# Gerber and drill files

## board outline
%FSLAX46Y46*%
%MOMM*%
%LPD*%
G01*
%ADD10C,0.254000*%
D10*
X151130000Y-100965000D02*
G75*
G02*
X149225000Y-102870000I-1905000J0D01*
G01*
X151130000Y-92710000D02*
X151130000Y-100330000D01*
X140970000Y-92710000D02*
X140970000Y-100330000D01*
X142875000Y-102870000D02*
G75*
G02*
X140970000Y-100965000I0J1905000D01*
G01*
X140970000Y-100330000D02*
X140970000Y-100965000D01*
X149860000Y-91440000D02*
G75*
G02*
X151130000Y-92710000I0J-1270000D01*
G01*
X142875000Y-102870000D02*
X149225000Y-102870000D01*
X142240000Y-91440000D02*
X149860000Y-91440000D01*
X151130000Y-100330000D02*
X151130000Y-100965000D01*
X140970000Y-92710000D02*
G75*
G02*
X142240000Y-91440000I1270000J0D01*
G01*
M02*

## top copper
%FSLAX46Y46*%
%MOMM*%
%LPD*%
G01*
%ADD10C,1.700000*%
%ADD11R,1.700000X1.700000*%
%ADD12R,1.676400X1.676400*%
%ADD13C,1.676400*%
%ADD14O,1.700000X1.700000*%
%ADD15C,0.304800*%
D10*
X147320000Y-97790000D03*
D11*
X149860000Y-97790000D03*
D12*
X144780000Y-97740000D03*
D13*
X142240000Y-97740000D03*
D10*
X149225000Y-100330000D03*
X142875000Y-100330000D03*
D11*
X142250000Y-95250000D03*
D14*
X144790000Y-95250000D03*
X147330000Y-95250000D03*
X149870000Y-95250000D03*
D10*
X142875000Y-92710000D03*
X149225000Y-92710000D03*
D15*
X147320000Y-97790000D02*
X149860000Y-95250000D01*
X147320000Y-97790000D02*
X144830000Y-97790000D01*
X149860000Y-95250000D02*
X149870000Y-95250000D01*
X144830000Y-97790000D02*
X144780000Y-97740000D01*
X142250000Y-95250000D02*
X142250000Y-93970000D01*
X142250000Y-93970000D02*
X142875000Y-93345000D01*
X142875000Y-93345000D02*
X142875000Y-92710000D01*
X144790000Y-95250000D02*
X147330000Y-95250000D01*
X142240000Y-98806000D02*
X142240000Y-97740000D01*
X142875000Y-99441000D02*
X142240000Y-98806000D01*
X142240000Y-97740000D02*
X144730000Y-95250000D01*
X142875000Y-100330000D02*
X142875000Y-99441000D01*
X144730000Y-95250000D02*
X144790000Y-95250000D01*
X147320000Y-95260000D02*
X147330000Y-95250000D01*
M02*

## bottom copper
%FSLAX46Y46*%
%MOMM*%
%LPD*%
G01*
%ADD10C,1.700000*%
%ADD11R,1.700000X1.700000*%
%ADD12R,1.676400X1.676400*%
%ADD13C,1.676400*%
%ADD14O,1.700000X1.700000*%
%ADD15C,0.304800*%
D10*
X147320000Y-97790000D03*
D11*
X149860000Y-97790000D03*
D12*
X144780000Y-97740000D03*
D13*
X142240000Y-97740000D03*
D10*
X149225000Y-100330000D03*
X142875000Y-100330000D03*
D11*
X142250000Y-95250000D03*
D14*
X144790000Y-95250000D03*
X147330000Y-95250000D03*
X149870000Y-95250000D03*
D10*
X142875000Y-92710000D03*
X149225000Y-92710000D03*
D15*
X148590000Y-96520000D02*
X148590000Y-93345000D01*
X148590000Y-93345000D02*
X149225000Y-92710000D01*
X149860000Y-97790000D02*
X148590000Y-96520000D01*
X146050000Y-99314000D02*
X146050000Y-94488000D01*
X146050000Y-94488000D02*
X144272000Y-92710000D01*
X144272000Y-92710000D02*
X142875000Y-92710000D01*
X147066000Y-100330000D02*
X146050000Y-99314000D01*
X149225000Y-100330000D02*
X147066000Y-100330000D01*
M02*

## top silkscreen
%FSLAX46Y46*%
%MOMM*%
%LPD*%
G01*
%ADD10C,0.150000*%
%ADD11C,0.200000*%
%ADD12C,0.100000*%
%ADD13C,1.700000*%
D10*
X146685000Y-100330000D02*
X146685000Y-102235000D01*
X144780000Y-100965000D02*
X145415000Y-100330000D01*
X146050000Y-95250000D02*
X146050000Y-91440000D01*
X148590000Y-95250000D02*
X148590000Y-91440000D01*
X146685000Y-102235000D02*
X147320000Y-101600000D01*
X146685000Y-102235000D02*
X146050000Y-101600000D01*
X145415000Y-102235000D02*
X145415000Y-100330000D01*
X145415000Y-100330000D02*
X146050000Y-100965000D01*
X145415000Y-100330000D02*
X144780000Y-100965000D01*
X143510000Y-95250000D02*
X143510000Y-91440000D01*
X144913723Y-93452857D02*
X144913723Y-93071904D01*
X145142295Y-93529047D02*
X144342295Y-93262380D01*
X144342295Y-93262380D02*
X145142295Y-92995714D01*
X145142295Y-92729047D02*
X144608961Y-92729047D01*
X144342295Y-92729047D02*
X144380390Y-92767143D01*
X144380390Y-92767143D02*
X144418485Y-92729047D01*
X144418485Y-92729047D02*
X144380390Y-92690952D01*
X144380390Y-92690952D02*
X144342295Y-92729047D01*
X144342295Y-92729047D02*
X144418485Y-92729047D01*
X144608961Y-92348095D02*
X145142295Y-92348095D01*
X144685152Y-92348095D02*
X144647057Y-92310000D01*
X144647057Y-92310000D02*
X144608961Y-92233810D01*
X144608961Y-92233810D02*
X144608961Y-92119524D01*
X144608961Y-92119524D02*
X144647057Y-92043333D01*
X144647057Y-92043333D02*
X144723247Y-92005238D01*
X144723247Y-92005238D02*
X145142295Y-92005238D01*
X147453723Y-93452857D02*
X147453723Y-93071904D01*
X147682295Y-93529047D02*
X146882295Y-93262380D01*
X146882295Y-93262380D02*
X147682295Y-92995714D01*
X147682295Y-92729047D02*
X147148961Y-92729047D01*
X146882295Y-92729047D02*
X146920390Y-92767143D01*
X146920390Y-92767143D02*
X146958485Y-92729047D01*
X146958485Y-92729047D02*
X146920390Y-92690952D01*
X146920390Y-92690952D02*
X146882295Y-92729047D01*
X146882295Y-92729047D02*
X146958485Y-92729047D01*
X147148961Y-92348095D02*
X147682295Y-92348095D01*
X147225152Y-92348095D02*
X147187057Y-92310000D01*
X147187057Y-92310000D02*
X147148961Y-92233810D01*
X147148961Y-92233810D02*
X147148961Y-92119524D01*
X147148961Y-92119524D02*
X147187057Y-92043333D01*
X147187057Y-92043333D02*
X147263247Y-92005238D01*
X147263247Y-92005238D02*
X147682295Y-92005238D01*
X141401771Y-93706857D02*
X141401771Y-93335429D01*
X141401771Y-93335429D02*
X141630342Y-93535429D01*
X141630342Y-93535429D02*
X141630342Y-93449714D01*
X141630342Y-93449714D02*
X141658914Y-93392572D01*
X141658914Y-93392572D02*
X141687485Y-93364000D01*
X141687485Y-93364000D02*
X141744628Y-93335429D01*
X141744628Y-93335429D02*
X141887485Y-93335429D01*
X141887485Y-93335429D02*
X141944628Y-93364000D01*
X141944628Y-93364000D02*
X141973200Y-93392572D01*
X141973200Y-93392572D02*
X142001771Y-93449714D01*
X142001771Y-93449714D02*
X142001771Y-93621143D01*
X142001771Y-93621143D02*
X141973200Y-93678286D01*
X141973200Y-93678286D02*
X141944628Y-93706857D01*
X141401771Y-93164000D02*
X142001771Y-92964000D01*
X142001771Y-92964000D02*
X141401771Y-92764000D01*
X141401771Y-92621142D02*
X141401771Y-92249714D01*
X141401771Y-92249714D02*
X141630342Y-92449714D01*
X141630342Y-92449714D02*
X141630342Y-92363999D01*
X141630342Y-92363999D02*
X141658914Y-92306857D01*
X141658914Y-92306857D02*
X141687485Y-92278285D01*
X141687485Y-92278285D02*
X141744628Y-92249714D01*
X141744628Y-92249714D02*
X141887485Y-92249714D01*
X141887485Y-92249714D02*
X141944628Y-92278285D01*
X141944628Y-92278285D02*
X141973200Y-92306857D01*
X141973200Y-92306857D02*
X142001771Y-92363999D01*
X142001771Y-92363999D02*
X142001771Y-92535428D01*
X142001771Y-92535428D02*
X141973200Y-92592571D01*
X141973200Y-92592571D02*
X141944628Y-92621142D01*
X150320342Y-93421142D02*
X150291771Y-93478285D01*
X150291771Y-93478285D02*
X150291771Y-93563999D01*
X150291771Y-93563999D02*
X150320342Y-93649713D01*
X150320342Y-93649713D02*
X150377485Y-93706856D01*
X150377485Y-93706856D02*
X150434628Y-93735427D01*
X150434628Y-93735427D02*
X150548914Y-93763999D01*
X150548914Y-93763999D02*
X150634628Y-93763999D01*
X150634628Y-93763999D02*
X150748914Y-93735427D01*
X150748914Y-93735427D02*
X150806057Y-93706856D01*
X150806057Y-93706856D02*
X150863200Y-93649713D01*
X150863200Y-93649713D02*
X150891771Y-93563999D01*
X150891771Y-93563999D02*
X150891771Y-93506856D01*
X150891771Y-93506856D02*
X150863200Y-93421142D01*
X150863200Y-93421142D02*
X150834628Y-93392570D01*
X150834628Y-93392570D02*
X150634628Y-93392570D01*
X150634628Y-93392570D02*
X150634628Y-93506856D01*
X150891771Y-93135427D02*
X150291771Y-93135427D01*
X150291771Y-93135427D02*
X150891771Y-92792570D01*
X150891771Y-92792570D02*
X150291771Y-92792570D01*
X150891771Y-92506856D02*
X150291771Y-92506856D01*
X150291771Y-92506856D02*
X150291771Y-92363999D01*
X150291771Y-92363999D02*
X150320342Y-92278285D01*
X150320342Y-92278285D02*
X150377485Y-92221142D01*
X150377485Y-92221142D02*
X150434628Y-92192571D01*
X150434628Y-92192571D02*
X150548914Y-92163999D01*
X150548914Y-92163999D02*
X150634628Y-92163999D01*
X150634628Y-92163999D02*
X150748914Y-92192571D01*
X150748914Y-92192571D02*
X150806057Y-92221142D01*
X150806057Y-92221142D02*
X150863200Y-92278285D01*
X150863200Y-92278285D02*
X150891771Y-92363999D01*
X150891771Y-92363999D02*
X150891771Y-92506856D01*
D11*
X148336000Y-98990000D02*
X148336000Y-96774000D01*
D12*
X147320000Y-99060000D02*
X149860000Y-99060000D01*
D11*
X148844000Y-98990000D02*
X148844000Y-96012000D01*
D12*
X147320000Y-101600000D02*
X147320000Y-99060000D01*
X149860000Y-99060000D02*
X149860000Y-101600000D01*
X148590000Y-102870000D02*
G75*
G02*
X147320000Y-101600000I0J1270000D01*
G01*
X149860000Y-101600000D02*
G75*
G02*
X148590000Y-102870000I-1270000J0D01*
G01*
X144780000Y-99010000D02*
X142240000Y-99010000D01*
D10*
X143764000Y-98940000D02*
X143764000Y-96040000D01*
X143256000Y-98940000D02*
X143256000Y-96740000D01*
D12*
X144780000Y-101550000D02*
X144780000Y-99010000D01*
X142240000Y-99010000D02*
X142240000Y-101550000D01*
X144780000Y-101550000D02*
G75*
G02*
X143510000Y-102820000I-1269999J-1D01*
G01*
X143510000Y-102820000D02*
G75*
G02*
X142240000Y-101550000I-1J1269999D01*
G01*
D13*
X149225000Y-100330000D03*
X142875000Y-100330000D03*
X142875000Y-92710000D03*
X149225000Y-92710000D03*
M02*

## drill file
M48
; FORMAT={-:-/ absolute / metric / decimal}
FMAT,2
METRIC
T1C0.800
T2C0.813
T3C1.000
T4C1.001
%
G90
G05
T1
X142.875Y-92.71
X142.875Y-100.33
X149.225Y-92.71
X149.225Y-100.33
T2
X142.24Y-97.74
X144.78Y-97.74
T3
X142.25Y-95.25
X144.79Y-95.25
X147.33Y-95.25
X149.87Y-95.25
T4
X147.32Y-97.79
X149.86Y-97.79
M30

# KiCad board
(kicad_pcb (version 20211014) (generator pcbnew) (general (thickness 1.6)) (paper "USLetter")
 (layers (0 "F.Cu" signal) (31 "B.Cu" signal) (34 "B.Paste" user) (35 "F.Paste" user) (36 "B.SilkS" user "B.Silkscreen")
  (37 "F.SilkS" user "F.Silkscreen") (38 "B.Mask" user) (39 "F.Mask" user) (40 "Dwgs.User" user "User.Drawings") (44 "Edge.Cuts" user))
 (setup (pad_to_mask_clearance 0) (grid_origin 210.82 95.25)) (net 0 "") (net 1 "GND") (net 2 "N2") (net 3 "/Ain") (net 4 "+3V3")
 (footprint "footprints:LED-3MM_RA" (layer "F.Cu") (at 147.32 97.79)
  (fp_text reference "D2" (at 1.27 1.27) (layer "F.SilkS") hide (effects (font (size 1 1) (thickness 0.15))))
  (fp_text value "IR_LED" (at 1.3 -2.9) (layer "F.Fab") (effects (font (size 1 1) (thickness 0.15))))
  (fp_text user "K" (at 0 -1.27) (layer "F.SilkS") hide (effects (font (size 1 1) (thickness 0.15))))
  (fp_line (start 1.016 1.2) (end 1.016 -1.016) (layer "F.SilkS") (width 0.2))
  (fp_line (start 0 1.27) (end 2.54 1.27) (layer "F.SilkS") (width 0.1))
  (fp_line (start 1.524 1.2) (end 1.524 -1.778) (layer "F.SilkS") (width 0.2))
  (fp_line (start 0 3.81) (end 0 1.27) (layer "F.SilkS") (width 0.1))
  (fp_line (start 2.54 1.27) (end 2.54 3.81) (layer "F.SilkS") (width 0.1))
  (fp_arc (start 1.27 5.08) (mid 0.371974 4.708026) (end 0 3.81) (layer "F.SilkS") (width 0.1))
  (fp_arc (start 2.54 3.81) (mid 2.168026 4.708026) (end 1.27 5.08) (layer "F.SilkS") (width 0.1))
  (pad "1" thru_hole circle (at 0 0 90) (size 1.7 1.7) (drill 1.00076) (layers *.Cu *.Mask) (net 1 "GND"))
  (pad "2" thru_hole rect (at 2.54 0) (size 1.7 1.7) (drill 1.00076) (layers *.Cu *.Mask) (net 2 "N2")))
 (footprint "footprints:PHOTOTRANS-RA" (layer "F.Cu") (at 143.51 97.74)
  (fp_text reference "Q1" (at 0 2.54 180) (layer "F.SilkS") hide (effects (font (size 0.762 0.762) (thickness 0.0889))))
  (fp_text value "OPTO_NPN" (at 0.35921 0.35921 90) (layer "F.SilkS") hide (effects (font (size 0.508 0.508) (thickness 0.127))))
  (fp_line (start 1.27 1.27) (end -1.27 1.27) (layer "F.SilkS") (width 0.1))
  (fp_line (start 0.254 1.2) (end 0.254 -1.7) (layer "F.SilkS") (width 0.15))
  (fp_line (start -0.254 1.2) (end -0.254 -1) (layer "F.SilkS") (width 0.15))
  (fp_line (start 1.27 3.81) (end 1.27 1.27) (layer "F.SilkS") (width 0.1))
  (fp_line (start -1.27 1.27) (end -1.27 3.81) (layer "F.SilkS") (width 0.1))
  (fp_arc (start 1.27 3.81) (mid 0.898026 4.708026) (end 0 5.08) (layer "F.SilkS") (width 0.1))
  (fp_arc (start 0 5.08) (mid -0.898026 4.708026) (end -1.27 3.81) (layer "F.SilkS") (width 0.1))
  (pad "1" thru_hole rect (at 1.27 0) (size 1.6764 1.6764) (drill 0.8128) (layers *.Cu *.Mask) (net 1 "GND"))
  (pad "3" thru_hole circle (at -1.27 0) (size 1.6764 1.6764) (drill 0.8128) (layers *.Cu *.Mask) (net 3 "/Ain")))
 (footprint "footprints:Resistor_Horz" (layer "B.Cu") (at 146.05 100.33 180)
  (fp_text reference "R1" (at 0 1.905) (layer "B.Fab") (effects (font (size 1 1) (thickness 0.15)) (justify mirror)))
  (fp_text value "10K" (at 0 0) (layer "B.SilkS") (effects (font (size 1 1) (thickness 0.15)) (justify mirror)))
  (pad "1" thru_hole circle (at -3.175 0 180) (size 1.7 1.7) (drill 0.8) (layers *.Cu *.SilkS *.Mask) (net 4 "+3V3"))
  (pad "2" thru_hole circle (at 3.175 0 180) (size 1.7 1.7) (drill 0.8) (layers *.Cu *.SilkS *.Mask) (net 3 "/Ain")))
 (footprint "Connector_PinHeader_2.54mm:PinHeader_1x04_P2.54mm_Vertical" (layer "B.Cu") (at 142.25 95.25 -90)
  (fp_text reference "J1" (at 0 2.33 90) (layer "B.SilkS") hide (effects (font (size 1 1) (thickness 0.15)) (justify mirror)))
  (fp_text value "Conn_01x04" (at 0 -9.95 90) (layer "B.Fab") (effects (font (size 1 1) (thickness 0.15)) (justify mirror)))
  (pad "1" thru_hole rect (at 0 0 270) (size 1.7 1.7) (drill 1) (layers *.Cu *.Mask) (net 4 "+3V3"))
  (pad "2" thru_hole oval (at 0 -2.54 270) (size 1.7 1.7) (drill 1) (layers *.Cu *.Mask) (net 3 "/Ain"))
  (pad "3" thru_hole oval (at 0 -5.08 270) (size 1.7 1.7) (drill 1) (layers *.Cu *.Mask) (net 3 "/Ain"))
  (pad "4" thru_hole oval (at 0 -7.62 270) (size 1.7 1.7) (drill 1) (layers *.Cu *.Mask) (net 1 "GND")))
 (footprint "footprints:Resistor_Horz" (layer "B.Cu") (at 146.05 92.71)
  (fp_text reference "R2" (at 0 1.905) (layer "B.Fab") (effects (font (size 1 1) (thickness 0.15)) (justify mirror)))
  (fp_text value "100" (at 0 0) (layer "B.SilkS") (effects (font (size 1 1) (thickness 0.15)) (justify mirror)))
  (pad "1" thru_hole circle (at -3.175 0) (size 1.7 1.7) (drill 0.8) (layers *.Cu *.SilkS *.Mask) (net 4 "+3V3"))
  (pad "2" thru_hole circle (at 3.175 0) (size 1.7 1.7) (drill 0.8) (layers *.Cu *.SilkS *.Mask) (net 2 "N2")))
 (gr_line (start 146.685 100.33) (end 146.685 102.235) (layer "F.SilkS") (width 0.15))
 (gr_line (start 144.78 100.965) (end 145.415 100.33) (layer "F.SilkS") (width 0.15))
 (gr_line (start 146.05 95.25) (end 146.05 91.44) (layer "F.SilkS") (width 0.15))
 (gr_line (start 148.59 95.25) (end 148.59 91.44) (layer "F.SilkS") (width 0.15))
 (gr_line (start 146.685 102.235) (end 147.32 101.6) (layer "F.SilkS") (width 0.15))
 (gr_line (start 146.685 102.235) (end 146.05 101.6) (layer "F.SilkS") (width 0.15))
 (gr_line (start 145.415 102.235) (end 145.415 100.33) (layer "F.SilkS") (width 0.15))
 (gr_line (start 145.415 100.33) (end 146.05 100.965) (layer "F.SilkS") (width 0.15))
 (gr_line (start 145.415 100.33) (end 144.78 100.965) (layer "F.SilkS") (width 0.15))
 (gr_line (start 143.51 95.25) (end 143.51 91.44) (layer "F.SilkS") (width 0.15))
 (gr_arc (start 151.13 100.965) (mid 150.572038 102.312038) (end 149.225 102.87) (layer "Edge.Cuts") (width 0.254))
 (gr_line (start 151.13 92.71) (end 151.13 100.33) (layer "Edge.Cuts") (width 0.254))
 (gr_line (start 140.97 92.71) (end 140.97 100.33) (layer "Edge.Cuts") (width 0.254))
 (gr_arc (start 142.875 102.87) (mid 141.527962 102.312038) (end 140.97 100.965) (layer "Edge.Cuts") (width 0.254))
 (gr_line (start 140.97 100.33) (end 140.97 100.965) (layer "Edge.Cuts") (width 0.254))
 (gr_arc (start 149.86 91.44) (mid 150.758026 91.811974) (end 151.13 92.71) (layer "Edge.Cuts") (width 0.254))
 (gr_line (start 142.875 102.87) (end 149.225 102.87) (layer "Edge.Cuts") (width 0.254))
 (gr_line (start 142.24 91.44) (end 149.86 91.44) (layer "Edge.Cuts") (width 0.254))
 (gr_line (start 151.13 100.33) (end 151.13 100.965) (layer "Edge.Cuts") (width 0.254))
 (gr_arc (start 140.97 92.71) (mid 141.341974 91.811974) (end 142.24 91.44) (layer "Edge.Cuts") (width 0.254))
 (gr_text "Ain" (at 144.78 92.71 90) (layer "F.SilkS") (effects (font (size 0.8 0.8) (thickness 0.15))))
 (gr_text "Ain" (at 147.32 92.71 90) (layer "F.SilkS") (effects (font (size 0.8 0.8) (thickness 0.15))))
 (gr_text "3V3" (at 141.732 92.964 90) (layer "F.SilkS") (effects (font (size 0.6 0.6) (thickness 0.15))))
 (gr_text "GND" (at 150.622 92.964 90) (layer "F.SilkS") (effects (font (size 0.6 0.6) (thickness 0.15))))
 (segment (start 147.32 97.79) (end 149.86 95.25) (width 0.3048) (layer "F.Cu") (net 1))
 (segment (start 147.32 97.79) (end 144.83 97.79) (width 0.3048) (layer "F.Cu") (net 1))
 (segment (start 149.86 95.25) (end 149.87 95.25) (width 0.3048) (layer "F.Cu") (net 1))
 (segment (start 144.83 97.79) (end 144.78 97.74) (width 0.3048) (layer "F.Cu") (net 1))
 (segment (start 148.59 96.52) (end 148.59 93.345) (width 0.3048) (layer "B.Cu") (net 2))
 (segment (start 148.59 93.345) (end 149.225 92.71) (width 0.3048) (layer "B.Cu") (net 2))
 (segment (start 149.86 97.79) (end 148.59 96.52) (width 0.3048) (layer "B.Cu") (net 2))
 (segment (start 142.25 95.25) (end 142.25 93.97) (width 0.3048) (layer "F.Cu") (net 4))
 (segment (start 142.25 93.97) (end 142.875 93.345) (width 0.3048) (layer "F.Cu") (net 4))
 (segment (start 142.875 93.345) (end 142.875 92.71) (width 0.3048) (layer "F.Cu") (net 4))
 (segment (start 146.05 99.314) (end 146.05 94.488) (width 0.3048) (layer "B.Cu") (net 4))
 (segment (start 146.05 94.488) (end 144.272 92.71) (width 0.3048) (layer "B.Cu") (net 4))
 (segment (start 144.272 92.71) (end 142.875 92.71) (width 0.3048) (layer "B.Cu") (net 4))
 (segment (start 147.066 100.33) (end 146.05 99.314) (width 0.3048) (layer "B.Cu") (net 4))
 (segment (start 149.225 100.33) (end 147.066 100.33) (width 0.3048) (layer "B.Cu") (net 4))
 (segment (start 144.79 95.25) (end 147.33 95.25) (width 0.3048) (layer "F.Cu") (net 3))
 (segment (start 142.24 98.806) (end 142.24 97.74) (width 0.3048) (layer "F.Cu") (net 3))
 (segment (start 142.875 99.441) (end 142.24 98.806) (width 0.3048) (layer "F.Cu") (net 3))
 (segment (start 142.24 97.74) (end 144.73 95.25) (width 0.3048) (layer "F.Cu") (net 3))
 (segment (start 142.875 100.33) (end 142.875 99.441) (width 0.3048) (layer "F.Cu") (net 3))
 (segment (start 144.73 95.25) (end 144.79 95.25) (width 0.3048) (layer "F.Cu") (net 3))
 (segment (start 147.32 95.26) (end 147.33 95.25) (width 0.3048) (layer "F.Cu") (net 3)))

